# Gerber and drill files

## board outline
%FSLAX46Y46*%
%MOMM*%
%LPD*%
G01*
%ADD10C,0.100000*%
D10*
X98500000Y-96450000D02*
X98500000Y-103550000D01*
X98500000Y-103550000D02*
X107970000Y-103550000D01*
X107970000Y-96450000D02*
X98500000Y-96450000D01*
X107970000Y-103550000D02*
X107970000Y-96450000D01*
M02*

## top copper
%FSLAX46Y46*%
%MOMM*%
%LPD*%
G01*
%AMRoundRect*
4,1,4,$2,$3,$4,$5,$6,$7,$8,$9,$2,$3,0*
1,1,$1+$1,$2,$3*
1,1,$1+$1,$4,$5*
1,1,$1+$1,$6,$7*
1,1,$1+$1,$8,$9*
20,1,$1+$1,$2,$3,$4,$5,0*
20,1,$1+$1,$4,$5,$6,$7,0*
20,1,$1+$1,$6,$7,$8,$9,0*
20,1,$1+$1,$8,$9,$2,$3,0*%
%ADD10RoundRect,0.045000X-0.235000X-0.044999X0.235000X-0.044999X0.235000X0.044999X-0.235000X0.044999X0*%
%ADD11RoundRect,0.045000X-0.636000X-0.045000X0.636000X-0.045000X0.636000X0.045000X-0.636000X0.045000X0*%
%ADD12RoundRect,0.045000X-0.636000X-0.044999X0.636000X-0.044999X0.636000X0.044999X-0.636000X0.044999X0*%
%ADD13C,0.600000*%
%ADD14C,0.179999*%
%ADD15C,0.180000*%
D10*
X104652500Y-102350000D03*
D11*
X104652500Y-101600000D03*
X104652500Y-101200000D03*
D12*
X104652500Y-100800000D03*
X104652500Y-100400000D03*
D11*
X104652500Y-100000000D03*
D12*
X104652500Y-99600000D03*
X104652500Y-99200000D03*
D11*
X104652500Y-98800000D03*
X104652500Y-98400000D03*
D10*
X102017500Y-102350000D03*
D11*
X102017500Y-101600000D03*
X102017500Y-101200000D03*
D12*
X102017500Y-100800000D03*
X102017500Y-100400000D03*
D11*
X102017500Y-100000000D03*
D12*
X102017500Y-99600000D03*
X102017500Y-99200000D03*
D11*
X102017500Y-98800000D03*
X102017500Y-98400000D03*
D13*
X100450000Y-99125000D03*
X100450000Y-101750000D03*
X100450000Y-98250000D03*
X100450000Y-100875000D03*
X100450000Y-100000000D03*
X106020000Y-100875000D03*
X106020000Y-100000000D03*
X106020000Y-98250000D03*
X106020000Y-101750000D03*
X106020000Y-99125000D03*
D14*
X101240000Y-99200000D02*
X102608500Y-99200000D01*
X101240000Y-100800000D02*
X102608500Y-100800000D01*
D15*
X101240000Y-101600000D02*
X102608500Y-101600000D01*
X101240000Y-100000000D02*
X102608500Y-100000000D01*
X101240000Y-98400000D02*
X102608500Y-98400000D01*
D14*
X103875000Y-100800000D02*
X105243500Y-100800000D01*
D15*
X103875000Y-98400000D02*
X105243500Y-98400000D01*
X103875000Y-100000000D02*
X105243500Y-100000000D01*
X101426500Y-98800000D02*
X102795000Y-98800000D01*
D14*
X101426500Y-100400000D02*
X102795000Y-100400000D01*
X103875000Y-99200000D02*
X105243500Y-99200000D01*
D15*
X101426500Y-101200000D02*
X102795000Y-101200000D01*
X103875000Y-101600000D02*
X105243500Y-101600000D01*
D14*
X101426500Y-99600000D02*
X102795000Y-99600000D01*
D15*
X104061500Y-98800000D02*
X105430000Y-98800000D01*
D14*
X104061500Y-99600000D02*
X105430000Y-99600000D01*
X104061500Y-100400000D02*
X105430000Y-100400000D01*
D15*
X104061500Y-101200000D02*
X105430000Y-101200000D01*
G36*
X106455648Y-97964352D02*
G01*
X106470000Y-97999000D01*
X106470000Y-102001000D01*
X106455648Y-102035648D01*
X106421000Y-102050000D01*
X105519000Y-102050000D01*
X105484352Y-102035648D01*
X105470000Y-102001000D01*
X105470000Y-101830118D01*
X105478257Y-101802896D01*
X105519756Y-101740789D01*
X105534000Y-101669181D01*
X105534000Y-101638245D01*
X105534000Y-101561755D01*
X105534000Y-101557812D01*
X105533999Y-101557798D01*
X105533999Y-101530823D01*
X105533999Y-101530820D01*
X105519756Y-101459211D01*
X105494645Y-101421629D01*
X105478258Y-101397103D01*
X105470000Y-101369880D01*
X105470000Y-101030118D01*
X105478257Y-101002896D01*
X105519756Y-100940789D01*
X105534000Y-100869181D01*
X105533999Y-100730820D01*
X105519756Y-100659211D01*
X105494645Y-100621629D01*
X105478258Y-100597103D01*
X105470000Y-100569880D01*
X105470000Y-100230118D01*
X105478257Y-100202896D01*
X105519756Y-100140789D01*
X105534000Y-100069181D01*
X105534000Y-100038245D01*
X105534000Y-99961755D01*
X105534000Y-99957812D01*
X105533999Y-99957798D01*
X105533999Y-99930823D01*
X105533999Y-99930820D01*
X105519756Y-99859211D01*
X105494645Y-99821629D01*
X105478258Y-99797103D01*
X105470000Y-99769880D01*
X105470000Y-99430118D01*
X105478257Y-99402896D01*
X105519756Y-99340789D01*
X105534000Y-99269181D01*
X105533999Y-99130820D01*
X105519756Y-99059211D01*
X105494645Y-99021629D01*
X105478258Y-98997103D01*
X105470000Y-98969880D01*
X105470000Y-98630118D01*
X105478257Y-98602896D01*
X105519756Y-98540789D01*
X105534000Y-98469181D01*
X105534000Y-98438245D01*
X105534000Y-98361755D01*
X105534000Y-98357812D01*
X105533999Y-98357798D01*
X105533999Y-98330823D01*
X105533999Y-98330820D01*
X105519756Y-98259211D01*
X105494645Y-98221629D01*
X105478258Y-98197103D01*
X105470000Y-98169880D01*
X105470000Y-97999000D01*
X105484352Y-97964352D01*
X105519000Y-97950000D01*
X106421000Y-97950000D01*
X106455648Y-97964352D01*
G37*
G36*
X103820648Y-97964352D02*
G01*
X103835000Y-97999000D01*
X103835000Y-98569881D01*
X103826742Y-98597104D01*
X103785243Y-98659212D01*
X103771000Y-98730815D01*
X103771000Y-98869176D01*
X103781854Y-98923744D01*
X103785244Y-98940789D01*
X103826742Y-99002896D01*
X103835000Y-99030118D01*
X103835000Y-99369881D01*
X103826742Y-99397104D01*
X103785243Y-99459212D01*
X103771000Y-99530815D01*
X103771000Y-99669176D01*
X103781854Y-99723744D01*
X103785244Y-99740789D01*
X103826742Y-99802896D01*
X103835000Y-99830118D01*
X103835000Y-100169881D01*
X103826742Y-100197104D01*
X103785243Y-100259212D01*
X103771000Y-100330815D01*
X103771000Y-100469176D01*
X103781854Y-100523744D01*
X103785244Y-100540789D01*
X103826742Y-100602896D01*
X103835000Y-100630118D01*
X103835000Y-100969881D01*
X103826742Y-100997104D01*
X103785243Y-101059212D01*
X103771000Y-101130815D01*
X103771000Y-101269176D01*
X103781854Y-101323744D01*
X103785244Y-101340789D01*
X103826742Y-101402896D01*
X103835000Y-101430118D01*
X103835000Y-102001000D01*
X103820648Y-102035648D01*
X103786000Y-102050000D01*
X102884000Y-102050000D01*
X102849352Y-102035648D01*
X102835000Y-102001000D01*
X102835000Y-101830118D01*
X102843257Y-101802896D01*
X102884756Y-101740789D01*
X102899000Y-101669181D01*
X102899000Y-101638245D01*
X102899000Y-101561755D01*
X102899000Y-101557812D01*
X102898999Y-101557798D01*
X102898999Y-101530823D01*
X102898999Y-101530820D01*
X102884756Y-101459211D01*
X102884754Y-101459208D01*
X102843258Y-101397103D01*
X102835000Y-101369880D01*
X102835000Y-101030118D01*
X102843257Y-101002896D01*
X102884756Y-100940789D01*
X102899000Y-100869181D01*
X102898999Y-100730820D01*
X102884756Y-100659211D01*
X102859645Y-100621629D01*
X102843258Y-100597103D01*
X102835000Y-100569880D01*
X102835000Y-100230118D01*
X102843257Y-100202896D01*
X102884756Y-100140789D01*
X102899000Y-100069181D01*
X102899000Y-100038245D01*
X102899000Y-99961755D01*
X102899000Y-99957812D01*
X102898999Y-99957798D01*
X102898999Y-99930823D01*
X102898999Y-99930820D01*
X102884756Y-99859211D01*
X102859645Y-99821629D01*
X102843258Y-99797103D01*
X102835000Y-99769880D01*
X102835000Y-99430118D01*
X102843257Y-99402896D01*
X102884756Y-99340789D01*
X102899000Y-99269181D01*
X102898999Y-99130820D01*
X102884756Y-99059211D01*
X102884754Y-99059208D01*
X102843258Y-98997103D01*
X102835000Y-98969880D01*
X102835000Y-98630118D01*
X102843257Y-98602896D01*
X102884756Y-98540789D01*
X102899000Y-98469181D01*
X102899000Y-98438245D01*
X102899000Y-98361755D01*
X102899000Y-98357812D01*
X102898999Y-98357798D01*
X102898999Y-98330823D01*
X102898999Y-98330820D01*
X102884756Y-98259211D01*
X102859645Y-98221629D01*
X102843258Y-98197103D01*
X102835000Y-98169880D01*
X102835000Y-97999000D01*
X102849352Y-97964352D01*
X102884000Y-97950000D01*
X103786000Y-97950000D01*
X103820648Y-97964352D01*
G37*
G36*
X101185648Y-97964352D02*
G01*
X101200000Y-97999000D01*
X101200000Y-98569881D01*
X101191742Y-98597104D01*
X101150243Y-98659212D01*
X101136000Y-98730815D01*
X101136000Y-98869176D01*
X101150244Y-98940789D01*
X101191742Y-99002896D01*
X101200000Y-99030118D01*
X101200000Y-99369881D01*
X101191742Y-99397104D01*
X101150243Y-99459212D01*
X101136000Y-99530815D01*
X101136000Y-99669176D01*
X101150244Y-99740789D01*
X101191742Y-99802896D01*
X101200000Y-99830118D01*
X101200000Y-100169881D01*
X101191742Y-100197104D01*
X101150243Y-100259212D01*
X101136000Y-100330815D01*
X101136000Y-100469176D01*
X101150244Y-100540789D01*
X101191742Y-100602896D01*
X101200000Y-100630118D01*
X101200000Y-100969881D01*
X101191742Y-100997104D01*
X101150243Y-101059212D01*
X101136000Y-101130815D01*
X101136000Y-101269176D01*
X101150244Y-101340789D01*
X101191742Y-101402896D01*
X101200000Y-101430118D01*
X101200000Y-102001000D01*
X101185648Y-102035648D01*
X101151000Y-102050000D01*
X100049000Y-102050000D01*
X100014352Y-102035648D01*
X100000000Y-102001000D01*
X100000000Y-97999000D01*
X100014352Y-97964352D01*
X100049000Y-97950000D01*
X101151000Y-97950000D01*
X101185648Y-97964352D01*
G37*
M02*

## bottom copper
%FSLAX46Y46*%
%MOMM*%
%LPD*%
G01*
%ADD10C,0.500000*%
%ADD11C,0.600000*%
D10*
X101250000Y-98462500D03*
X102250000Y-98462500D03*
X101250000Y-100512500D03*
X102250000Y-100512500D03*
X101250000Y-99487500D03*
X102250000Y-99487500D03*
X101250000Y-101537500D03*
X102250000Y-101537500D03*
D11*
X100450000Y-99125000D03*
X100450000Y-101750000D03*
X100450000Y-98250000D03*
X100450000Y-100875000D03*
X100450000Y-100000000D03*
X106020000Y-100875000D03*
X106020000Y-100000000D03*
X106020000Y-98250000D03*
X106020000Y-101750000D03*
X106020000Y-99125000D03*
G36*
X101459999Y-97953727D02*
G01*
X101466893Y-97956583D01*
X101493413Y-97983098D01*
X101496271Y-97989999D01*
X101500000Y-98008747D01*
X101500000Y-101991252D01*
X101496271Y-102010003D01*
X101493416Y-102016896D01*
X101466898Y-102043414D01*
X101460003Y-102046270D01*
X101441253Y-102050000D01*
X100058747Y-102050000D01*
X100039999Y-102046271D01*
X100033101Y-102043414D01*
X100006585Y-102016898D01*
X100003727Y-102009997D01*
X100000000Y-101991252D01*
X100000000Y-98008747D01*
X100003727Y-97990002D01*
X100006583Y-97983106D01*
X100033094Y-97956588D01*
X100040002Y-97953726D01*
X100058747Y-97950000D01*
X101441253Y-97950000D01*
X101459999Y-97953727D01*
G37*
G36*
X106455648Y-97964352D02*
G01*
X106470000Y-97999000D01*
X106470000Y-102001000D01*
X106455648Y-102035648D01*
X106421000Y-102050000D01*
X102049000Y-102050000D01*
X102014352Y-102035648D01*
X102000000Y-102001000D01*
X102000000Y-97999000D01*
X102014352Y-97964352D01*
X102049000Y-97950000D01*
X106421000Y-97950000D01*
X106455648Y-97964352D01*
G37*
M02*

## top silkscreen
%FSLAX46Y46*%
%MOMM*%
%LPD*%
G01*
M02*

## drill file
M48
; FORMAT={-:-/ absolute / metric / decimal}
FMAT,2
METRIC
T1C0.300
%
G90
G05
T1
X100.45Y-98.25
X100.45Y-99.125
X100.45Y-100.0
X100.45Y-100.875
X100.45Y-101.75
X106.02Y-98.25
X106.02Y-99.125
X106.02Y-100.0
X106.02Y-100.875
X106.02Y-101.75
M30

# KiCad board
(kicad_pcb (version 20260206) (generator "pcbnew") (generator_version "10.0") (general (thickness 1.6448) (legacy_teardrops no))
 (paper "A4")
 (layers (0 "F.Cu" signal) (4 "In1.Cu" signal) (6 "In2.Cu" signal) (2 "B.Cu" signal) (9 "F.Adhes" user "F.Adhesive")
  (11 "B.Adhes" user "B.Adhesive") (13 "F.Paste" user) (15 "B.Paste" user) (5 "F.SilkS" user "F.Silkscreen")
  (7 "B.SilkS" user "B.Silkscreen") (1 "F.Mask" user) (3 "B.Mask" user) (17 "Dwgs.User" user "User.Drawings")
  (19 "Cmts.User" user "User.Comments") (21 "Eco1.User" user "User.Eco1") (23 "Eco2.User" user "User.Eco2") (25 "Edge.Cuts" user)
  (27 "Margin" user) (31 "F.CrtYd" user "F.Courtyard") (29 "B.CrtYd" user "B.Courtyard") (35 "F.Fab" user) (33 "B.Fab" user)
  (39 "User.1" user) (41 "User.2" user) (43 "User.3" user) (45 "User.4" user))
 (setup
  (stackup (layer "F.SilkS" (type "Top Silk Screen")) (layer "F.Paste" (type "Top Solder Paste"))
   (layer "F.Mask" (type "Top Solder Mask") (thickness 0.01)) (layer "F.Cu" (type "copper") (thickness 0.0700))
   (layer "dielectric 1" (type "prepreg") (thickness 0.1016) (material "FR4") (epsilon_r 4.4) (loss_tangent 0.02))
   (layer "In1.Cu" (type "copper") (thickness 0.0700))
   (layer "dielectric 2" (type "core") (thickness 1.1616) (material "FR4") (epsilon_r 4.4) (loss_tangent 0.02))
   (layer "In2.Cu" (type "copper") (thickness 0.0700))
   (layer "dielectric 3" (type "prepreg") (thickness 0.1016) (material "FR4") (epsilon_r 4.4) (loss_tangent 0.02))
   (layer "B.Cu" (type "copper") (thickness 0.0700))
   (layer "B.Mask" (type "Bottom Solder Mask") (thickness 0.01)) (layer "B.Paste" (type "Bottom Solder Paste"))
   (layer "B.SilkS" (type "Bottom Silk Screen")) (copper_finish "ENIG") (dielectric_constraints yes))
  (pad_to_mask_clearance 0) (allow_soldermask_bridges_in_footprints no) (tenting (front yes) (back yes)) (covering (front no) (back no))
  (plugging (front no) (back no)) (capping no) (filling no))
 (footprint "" (layer "F.Cu") (at 0 0)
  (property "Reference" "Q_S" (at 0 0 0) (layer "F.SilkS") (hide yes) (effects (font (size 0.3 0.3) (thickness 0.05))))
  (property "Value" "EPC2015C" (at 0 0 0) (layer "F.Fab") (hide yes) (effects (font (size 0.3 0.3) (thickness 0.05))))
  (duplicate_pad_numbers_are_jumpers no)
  (pad "1" smd roundrect (at 104.6525 102.35) (size 0.56 0.179999) (layers "F.Cu" "F.Mask" "F.Paste") (roundrect_rratio 0.25) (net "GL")
   (thermal_bridge_angle 45))
  (pad "3" smd roundrect (at 104.6525 101.6) (size 1.362 0.18) (layers "F.Cu" "F.Mask" "F.Paste") (roundrect_rratio 0.25) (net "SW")
   (thermal_bridge_angle 45))
  (pad "4" smd roundrect (at 104.6525 101.2) (size 1.362 0.18) (layers "F.Cu" "F.Mask" "F.Paste") (roundrect_rratio 0.25) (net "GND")
   (thermal_bridge_angle 45))
  (pad "5" smd roundrect (at 104.6525 100.8) (size 1.362 0.179999) (layers "F.Cu" "F.Mask" "F.Paste") (roundrect_rratio 0.25) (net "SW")
   (thermal_bridge_angle 45))
  (pad "6" smd roundrect (at 104.6525 100.4) (size 1.362 0.179999) (layers "F.Cu" "F.Mask" "F.Paste") (roundrect_rratio 0.25) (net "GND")
   (thermal_bridge_angle 45))
  (pad "7" smd roundrect (at 104.6525 100) (size 1.362 0.18) (layers "F.Cu" "F.Mask" "F.Paste") (roundrect_rratio 0.25) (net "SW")
   (thermal_bridge_angle 45))
  (pad "8" smd roundrect (at 104.6525 99.6) (size 1.362 0.179999) (layers "F.Cu" "F.Mask" "F.Paste") (roundrect_rratio 0.25) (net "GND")
   (thermal_bridge_angle 45))
  (pad "9" smd roundrect (at 104.6525 99.2) (size 1.362 0.179999) (layers "F.Cu" "F.Mask" "F.Paste") (roundrect_rratio 0.25) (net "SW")
   (thermal_bridge_angle 45))
  (pad "10" smd roundrect (at 104.6525 98.8) (size 1.362 0.18) (layers "F.Cu" "F.Mask" "F.Paste") (roundrect_rratio 0.25) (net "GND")
   (thermal_bridge_angle 45))
  (pad "11" smd roundrect (at 104.6525 98.4) (size 1.362 0.18) (layers "F.Cu" "F.Mask" "F.Paste") (roundrect_rratio 0.25) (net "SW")
   (thermal_bridge_angle 45)))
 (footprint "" (layer "F.Cu") (at 0 0)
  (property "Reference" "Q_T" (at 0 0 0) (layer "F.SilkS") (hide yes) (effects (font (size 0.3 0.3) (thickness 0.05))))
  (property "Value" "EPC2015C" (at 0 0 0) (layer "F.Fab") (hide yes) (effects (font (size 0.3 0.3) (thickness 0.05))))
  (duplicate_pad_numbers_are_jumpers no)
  (pad "1" smd roundrect (at 102.0175 102.35) (size 0.56 0.179999) (layers "F.Cu" "F.Mask" "F.Paste") (roundrect_rratio 0.25) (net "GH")
   (thermal_bridge_angle 45))
  (pad "3" smd roundrect (at 102.0175 101.6) (size 1.362 0.18) (layers "F.Cu" "F.Mask" "F.Paste") (roundrect_rratio 0.25) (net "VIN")
   (thermal_bridge_angle 45))
  (pad "4" smd roundrect (at 102.0175 101.2) (size 1.362 0.18) (layers "F.Cu" "F.Mask" "F.Paste") (roundrect_rratio 0.25) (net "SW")
   (thermal_bridge_angle 45))
  (pad "5" smd roundrect (at 102.0175 100.8) (size 1.362 0.179999) (layers "F.Cu" "F.Mask" "F.Paste") (roundrect_rratio 0.25) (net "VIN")
   (thermal_bridge_angle 45))
  (pad "6" smd roundrect (at 102.0175 100.4) (size 1.362 0.179999) (layers "F.Cu" "F.Mask" "F.Paste") (roundrect_rratio 0.25) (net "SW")
   (thermal_bridge_angle 45))
  (pad "7" smd roundrect (at 102.0175 100) (size 1.362 0.18) (layers "F.Cu" "F.Mask" "F.Paste") (roundrect_rratio 0.25) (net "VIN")
   (thermal_bridge_angle 45))
  (pad "8" smd roundrect (at 102.0175 99.6) (size 1.362 0.179999) (layers "F.Cu" "F.Mask" "F.Paste") (roundrect_rratio 0.25) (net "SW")
   (thermal_bridge_angle 45))
  (pad "9" smd roundrect (at 102.0175 99.2) (size 1.362 0.179999) (layers "F.Cu" "F.Mask" "F.Paste") (roundrect_rratio 0.25) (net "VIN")
   (thermal_bridge_angle 45))
  (pad "10" smd roundrect (at 102.0175 98.8) (size 1.362 0.18) (layers "F.Cu" "F.Mask" "F.Paste") (roundrect_rratio 0.25) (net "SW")
   (thermal_bridge_angle 45))
  (pad "11" smd roundrect (at 102.0175 98.4) (size 1.362 0.18) (layers "F.Cu" "F.Mask" "F.Paste") (roundrect_rratio 0.25) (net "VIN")
   (thermal_bridge_angle 45)))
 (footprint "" (layer "B.Cu") (at 101.75 98.4625)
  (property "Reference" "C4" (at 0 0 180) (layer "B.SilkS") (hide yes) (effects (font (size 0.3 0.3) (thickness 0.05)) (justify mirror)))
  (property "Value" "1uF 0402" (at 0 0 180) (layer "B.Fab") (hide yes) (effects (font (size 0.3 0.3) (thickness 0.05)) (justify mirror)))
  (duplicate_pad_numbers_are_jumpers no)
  (pad "1" smd circle (at -0.5 0) (size 0.5 0.5) (layers "B.Cu" "B.Mask" "B.Paste") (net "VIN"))
  (pad "2" smd circle (at 0.5 0) (size 0.5 0.5) (layers "B.Cu" "B.Mask" "B.Paste") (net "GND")))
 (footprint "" (layer "B.Cu") (at 101.75 100.5125)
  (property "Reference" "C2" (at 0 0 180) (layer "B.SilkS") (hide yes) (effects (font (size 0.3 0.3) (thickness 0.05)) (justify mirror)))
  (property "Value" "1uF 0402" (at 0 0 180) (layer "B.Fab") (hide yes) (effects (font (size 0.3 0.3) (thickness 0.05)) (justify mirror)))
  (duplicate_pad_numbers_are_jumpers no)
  (pad "1" smd circle (at -0.5 0) (size 0.5 0.5) (layers "B.Cu" "B.Mask" "B.Paste") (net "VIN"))
  (pad "2" smd circle (at 0.5 0) (size 0.5 0.5) (layers "B.Cu" "B.Mask" "B.Paste") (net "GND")))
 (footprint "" (layer "B.Cu") (at 101.75 99.4875)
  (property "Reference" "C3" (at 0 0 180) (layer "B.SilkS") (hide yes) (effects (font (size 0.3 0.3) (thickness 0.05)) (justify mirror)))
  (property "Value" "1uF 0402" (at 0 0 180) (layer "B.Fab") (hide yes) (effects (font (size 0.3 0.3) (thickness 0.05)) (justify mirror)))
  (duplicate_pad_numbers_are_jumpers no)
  (pad "1" smd circle (at -0.5 0) (size 0.5 0.5) (layers "B.Cu" "B.Mask" "B.Paste") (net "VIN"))
  (pad "2" smd circle (at 0.5 0) (size 0.5 0.5) (layers "B.Cu" "B.Mask" "B.Paste") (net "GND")))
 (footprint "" (layer "B.Cu") (at 101.75 101.5375)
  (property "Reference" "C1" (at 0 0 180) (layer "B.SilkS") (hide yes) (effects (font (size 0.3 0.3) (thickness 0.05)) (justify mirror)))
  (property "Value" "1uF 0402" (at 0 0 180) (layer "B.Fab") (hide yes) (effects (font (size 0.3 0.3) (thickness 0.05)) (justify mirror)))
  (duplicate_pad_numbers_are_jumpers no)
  (pad "1" smd circle (at -0.5 0) (size 0.5 0.5) (layers "B.Cu" "B.Mask" "B.Paste") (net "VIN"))
  (pad "2" smd circle (at 0.5 0) (size 0.5 0.5) (layers "B.Cu" "B.Mask" "B.Paste") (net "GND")))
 (gr_line (start 98.5 96.45) (end 98.5 103.55) (stroke (width 0.1) (type default)) (layer "Edge.Cuts"))
 (gr_line (start 98.5 103.55) (end 107.97 103.55) (stroke (width 0.1) (type default)) (layer "Edge.Cuts"))
 (gr_line (start 107.97 96.45) (end 98.5 96.45) (stroke (width 0.1) (type default)) (layer "Edge.Cuts"))
 (gr_line (start 107.97 103.55) (end 107.97 96.45) (stroke (width 0.1) (type default)) (layer "Edge.Cuts"))
 (segment (start 101.24 99.2) (end 102.6085 99.2) (width 0.179999) (layer "F.Cu") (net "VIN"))
 (segment (start 101.24 100.8) (end 102.6085 100.8) (width 0.179999) (layer "F.Cu") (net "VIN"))
 (segment (start 101.24 101.6) (end 102.6085 101.6) (width 0.18) (layer "F.Cu") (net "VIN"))
 (segment (start 101.24 100) (end 102.6085 100) (width 0.18) (layer "F.Cu") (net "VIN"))
 (segment (start 101.24 98.4) (end 102.6085 98.4) (width 0.18) (layer "F.Cu") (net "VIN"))
 (via (at 100.45 99.125) (size 0.6) (drill 0.3) (layers "F.Cu" "B.Cu") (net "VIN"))
 (via (at 100.45 101.75) (size 0.6) (drill 0.3) (layers "F.Cu" "B.Cu") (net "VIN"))
 (via (at 100.45 98.25) (size 0.6) (drill 0.3) (layers "F.Cu" "B.Cu") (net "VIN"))
 (via (at 100.45 100.875) (size 0.6) (drill 0.3) (layers "F.Cu" "B.Cu") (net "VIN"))
 (via (at 100.45 100) (size 0.6) (drill 0.3) (layers "F.Cu" "B.Cu") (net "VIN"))
 (segment (start 103.875 100.8) (end 105.2435 100.8) (width 0.179999) (layer "F.Cu") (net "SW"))
 (segment (start 103.875 98.4) (end 105.2435 98.4) (width 0.18) (layer "F.Cu") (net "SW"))
 (segment (start 103.875 100) (end 105.2435 100) (width 0.18) (layer "F.Cu") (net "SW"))
 (segment (start 101.4265 98.8) (end 102.795 98.8) (width 0.18) (layer "F.Cu") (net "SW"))
 (segment (start 101.4265 100.4) (end 102.795 100.4) (width 0.179999) (layer "F.Cu") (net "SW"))
 (segment (start 103.875 99.2) (end 105.2435 99.2) (width 0.179999) (layer "F.Cu") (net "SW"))
 (segment (start 101.4265 101.2) (end 102.795 101.2) (width 0.18) (layer "F.Cu") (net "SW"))
 (segment (start 103.875 101.6) (end 105.2435 101.6) (width 0.18) (layer "F.Cu") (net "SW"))
 (segment (start 101.4265 99.6) (end 102.795 99.6) (width 0.179999) (layer "F.Cu") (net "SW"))
 (segment (start 104.0615 98.8) (end 105.43 98.8) (width 0.18) (layer "F.Cu") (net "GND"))
 (segment (start 104.0615 99.6) (end 105.43 99.6) (width 0.179999) (layer "F.Cu") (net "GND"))
 (segment (start 104.0615 100.4) (end 105.43 100.4) (width 0.179999) (layer "F.Cu") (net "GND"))
 (segment (start 104.0615 101.2) (end 105.43 101.2) (width 0.18) (layer "F.Cu") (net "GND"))
 (via (at 106.02 100.875) (size 0.6) (drill 0.3) (layers "F.Cu" "B.Cu") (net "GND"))
 (via (at 106.02 100) (size 0.6) (drill 0.3) (layers "F.Cu" "B.Cu") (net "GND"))
 (via (at 106.02 98.25) (size 0.6) (drill 0.3) (layers "F.Cu" "B.Cu") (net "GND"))
 (via (at 106.02 101.75) (size 0.6) (drill 0.3) (layers "F.Cu" "B.Cu") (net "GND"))
 (via (at 106.02 99.125) (size 0.6) (drill 0.3) (layers "F.Cu" "B.Cu") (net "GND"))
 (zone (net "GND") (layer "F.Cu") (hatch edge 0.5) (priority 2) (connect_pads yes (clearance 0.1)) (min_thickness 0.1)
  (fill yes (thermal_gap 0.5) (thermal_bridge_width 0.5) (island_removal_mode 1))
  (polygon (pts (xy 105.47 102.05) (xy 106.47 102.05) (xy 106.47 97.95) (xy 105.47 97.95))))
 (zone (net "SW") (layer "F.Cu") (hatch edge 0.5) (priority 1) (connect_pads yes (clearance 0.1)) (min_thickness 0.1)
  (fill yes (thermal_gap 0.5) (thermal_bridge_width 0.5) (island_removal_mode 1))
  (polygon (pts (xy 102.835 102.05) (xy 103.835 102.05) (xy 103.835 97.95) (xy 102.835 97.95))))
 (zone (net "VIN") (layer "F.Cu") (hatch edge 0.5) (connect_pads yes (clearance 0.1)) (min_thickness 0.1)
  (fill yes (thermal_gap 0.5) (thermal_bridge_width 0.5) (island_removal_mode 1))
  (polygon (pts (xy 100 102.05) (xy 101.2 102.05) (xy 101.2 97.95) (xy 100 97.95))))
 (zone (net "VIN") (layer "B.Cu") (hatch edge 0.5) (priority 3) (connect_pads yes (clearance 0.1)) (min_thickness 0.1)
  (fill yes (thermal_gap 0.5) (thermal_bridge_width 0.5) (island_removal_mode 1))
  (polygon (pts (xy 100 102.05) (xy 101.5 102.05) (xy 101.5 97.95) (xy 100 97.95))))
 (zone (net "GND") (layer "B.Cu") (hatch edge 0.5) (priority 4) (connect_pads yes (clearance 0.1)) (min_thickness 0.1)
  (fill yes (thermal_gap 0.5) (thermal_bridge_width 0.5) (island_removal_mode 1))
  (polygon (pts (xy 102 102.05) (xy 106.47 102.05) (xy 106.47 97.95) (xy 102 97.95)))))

